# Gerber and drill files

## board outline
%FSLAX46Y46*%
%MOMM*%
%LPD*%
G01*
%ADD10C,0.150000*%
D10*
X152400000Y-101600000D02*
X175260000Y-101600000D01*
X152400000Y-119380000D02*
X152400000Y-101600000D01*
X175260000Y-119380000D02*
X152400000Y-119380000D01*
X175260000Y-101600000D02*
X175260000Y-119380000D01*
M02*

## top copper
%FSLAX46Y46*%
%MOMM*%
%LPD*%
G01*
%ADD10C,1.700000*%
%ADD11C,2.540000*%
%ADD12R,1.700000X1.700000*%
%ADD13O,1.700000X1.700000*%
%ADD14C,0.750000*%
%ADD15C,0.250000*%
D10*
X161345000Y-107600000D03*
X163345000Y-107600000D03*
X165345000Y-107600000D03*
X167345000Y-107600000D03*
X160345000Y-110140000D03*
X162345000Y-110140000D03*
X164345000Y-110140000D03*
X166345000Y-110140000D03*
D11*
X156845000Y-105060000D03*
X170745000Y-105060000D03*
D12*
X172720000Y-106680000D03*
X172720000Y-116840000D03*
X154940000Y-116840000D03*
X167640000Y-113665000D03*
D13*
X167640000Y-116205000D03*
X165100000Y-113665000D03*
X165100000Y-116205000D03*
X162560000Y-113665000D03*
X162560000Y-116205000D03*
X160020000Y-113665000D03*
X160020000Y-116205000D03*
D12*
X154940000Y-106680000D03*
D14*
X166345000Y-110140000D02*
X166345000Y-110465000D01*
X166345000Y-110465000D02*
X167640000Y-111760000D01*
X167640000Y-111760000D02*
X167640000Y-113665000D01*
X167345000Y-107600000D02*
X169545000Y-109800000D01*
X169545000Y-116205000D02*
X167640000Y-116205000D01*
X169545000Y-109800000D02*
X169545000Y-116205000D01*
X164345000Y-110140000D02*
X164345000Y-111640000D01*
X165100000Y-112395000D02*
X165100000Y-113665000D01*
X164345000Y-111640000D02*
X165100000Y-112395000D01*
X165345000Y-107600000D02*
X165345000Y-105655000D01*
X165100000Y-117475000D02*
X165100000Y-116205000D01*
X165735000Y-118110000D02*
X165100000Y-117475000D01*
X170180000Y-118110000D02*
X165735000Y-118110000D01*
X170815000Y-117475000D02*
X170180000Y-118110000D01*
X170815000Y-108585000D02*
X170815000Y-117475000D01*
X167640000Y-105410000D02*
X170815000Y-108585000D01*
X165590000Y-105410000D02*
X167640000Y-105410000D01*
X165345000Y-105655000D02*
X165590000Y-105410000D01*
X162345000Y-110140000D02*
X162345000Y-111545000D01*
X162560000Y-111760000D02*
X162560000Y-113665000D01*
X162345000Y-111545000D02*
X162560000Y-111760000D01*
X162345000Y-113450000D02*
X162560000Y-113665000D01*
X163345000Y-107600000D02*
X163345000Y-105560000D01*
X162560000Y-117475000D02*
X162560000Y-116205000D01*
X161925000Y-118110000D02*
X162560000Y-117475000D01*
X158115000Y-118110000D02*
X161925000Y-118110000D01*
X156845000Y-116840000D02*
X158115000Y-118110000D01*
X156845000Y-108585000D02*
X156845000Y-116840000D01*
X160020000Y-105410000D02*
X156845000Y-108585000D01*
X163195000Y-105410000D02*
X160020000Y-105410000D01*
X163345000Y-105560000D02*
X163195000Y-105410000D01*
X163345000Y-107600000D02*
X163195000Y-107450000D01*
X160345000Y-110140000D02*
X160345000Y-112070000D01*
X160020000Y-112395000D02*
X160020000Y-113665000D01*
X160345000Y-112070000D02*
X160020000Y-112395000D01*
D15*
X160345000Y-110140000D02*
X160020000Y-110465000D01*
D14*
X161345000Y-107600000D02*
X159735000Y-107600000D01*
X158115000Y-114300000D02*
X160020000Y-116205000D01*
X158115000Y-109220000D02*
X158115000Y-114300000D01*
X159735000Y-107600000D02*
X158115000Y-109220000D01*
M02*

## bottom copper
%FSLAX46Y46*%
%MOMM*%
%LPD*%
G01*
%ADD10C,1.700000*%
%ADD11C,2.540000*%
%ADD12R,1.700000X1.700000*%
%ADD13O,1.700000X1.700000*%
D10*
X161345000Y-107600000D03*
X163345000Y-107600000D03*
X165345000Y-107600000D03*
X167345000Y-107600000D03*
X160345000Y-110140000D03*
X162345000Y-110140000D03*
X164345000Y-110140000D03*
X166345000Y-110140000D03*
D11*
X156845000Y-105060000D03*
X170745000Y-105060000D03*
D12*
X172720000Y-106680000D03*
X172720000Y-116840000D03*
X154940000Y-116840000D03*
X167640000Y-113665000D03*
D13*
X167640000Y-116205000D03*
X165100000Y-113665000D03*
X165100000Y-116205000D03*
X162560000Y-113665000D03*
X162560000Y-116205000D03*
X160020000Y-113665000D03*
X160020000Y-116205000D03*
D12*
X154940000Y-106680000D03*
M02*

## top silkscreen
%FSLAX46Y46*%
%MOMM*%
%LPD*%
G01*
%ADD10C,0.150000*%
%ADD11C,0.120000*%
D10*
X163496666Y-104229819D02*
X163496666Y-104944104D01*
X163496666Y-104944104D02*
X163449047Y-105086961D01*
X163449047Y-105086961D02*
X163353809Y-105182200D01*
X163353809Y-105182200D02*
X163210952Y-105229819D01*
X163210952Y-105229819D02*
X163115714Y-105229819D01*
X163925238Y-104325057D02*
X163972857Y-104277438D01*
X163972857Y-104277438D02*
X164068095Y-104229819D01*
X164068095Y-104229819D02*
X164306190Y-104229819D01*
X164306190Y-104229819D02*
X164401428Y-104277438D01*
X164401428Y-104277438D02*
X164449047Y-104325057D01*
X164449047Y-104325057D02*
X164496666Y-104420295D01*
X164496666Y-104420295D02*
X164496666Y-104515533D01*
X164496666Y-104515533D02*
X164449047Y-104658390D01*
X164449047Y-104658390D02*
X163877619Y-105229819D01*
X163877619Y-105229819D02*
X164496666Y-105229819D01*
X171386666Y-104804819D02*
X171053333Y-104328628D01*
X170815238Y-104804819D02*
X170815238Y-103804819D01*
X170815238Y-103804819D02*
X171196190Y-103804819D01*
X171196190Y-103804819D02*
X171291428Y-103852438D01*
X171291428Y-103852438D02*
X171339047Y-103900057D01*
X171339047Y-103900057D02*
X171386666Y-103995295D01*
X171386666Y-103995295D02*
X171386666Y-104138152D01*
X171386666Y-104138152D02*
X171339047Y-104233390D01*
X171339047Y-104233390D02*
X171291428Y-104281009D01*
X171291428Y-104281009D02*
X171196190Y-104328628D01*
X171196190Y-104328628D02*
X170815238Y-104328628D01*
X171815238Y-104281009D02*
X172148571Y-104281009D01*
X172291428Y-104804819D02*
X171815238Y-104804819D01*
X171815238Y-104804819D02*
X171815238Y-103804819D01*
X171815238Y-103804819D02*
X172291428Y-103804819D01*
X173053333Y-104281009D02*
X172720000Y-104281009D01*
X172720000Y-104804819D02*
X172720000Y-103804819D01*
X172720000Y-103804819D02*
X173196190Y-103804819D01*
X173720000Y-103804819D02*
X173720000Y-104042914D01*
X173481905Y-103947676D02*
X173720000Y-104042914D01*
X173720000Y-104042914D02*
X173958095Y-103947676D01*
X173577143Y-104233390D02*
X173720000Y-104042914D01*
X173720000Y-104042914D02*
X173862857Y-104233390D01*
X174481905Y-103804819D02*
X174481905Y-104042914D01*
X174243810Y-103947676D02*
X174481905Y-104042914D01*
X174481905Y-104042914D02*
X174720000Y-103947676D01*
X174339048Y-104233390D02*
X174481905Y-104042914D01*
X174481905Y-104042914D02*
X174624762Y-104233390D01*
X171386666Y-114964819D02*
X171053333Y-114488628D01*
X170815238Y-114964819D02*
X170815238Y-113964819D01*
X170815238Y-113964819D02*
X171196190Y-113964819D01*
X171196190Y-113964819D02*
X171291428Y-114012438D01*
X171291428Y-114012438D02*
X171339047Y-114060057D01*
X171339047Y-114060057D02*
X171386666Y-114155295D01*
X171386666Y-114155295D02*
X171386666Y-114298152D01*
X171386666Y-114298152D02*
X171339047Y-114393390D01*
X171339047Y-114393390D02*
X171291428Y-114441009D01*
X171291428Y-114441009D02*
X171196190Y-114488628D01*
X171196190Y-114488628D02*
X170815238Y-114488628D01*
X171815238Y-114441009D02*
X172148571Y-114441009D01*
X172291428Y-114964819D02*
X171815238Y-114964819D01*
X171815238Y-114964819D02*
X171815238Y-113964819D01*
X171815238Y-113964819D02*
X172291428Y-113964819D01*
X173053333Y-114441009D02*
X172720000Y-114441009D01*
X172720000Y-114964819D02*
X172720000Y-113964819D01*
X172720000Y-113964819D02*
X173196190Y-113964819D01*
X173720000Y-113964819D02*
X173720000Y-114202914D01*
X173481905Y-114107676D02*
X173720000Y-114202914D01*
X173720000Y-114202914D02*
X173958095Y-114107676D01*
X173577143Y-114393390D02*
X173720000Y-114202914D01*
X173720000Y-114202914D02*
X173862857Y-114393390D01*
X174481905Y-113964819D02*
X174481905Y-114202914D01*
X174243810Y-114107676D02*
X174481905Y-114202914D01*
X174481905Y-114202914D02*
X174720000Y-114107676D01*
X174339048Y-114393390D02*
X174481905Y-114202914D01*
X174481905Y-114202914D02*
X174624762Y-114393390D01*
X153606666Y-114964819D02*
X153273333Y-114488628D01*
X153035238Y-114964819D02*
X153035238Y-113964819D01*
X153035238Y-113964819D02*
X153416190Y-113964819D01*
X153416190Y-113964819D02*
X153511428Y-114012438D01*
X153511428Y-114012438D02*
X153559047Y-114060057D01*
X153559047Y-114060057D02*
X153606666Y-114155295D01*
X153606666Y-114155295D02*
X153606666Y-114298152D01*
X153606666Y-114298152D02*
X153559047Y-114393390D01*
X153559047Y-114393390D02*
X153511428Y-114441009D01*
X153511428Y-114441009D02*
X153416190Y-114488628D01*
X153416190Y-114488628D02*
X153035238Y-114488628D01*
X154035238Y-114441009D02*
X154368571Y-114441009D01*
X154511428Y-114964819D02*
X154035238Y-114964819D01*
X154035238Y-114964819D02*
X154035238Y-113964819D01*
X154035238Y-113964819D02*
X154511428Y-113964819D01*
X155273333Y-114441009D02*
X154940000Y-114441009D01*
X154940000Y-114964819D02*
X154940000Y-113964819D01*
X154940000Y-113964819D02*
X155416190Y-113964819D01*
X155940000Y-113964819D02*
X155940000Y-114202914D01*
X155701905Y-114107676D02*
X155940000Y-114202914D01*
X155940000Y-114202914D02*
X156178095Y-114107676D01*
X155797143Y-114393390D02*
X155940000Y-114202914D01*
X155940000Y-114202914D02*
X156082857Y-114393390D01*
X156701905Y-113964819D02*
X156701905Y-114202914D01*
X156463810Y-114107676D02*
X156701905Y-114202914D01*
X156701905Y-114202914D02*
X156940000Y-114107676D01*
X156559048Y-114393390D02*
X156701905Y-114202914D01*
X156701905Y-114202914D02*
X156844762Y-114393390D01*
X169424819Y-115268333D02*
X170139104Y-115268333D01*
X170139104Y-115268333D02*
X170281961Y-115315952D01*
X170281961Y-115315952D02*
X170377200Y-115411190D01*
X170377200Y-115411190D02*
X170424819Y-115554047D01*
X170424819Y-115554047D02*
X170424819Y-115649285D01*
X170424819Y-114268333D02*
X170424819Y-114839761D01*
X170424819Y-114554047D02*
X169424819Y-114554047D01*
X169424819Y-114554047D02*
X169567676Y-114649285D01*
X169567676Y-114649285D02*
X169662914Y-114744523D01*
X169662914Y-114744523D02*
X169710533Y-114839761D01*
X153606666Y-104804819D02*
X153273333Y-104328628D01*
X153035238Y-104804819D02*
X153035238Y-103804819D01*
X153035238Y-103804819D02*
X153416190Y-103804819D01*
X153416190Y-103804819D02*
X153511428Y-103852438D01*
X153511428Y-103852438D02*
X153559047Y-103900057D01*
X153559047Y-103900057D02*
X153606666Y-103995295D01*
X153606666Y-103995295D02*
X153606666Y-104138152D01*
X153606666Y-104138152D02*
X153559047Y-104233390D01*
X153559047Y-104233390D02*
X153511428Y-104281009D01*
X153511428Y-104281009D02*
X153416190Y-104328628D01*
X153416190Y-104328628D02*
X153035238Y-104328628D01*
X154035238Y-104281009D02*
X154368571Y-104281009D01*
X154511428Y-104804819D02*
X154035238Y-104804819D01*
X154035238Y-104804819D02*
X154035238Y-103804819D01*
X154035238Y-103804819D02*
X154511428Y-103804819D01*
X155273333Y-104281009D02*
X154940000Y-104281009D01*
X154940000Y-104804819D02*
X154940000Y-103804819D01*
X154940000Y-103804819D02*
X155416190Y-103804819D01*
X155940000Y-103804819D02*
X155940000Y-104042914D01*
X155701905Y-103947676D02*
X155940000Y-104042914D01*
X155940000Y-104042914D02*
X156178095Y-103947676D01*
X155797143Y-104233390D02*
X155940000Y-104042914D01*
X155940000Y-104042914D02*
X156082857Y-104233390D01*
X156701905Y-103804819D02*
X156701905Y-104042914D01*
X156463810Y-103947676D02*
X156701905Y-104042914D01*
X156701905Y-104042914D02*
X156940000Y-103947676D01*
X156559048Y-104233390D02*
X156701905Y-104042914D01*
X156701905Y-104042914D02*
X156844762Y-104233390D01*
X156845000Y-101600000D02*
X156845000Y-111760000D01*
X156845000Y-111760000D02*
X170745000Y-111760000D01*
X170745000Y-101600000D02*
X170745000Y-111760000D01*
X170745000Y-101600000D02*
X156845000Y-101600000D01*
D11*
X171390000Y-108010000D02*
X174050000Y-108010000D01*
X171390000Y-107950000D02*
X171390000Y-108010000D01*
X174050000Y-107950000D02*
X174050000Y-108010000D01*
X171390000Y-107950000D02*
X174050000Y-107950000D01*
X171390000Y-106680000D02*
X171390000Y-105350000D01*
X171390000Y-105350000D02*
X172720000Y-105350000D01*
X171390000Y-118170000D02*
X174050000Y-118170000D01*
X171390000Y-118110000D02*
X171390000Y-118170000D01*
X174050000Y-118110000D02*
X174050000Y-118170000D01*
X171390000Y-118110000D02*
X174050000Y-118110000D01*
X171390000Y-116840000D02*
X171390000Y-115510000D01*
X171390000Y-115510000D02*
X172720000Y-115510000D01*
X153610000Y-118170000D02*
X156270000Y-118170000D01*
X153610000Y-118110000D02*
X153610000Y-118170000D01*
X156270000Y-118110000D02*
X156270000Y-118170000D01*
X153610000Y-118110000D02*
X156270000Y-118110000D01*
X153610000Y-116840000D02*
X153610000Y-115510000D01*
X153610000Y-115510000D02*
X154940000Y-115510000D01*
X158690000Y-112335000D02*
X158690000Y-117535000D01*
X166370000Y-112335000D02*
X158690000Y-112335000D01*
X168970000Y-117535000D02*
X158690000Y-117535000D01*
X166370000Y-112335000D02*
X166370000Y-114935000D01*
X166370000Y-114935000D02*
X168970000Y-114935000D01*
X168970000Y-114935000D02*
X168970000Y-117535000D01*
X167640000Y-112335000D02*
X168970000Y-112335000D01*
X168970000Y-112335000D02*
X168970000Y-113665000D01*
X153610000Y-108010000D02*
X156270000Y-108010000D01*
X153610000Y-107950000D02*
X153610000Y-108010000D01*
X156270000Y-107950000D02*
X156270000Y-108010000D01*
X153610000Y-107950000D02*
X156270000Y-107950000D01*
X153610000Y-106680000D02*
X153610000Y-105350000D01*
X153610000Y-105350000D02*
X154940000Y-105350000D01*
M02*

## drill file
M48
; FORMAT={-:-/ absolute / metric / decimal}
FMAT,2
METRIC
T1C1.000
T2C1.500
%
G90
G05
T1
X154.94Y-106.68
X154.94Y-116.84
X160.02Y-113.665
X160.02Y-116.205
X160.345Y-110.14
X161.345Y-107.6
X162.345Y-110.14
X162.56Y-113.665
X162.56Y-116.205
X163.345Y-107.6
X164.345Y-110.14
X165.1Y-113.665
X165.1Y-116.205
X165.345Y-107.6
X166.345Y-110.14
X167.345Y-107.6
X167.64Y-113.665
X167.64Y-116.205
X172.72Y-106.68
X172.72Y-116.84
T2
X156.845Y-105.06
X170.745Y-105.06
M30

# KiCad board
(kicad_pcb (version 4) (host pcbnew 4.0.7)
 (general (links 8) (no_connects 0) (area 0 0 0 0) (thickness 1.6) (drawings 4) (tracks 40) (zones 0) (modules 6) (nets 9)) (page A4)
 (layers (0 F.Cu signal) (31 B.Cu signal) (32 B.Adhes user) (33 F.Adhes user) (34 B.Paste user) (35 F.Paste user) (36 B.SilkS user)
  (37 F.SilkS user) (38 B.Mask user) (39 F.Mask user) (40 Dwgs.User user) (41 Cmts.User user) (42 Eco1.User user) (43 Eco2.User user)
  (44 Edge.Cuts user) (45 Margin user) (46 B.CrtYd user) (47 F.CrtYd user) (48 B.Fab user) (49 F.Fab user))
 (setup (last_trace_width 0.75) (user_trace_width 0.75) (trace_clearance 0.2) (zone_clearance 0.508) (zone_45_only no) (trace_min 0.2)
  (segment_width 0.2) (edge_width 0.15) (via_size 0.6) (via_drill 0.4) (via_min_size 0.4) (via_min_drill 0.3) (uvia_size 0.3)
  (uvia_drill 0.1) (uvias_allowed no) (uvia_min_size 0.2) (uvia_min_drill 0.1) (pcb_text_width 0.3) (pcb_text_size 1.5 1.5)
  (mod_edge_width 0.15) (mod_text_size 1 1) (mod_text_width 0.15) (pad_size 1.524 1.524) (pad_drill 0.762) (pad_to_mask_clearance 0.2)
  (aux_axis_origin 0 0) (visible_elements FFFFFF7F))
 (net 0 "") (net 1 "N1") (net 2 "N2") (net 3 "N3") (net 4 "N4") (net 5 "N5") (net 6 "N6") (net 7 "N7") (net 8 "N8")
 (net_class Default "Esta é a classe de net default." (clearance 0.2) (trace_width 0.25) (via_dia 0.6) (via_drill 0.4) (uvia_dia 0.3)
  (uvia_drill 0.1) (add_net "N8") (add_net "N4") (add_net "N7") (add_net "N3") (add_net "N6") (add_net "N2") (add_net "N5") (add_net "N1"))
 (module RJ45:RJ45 (layer F.Cu) (at 156.845 101.6)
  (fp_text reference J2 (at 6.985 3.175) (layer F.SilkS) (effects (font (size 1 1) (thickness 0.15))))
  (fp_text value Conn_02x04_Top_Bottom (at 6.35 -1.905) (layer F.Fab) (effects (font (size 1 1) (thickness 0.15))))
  (fp_line (start 0 0) (end 0 10.16) (layer F.SilkS) (width 0.15))
  (fp_line (start 0 10.16) (end 13.9 10.16) (layer F.SilkS) (width 0.15))
  (fp_line (start 13.9 0) (end 13.9 10.16) (layer F.SilkS) (width 0.15))
  (fp_line (start 13.9 0) (end 0 0) (layer F.SilkS) (width 0.15))
  (pad 1 thru_hole circle (at 4.5 6) (size 1.7 1.7) (drill 1) (layers *.Cu *.Mask) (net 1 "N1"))
  (pad 2 thru_hole circle (at 6.5 6) (size 1.7 1.7) (drill 1) (layers *.Cu *.Mask) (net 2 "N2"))
  (pad 3 thru_hole circle (at 8.5 6) (size 1.7 1.7) (drill 1) (layers *.Cu *.Mask) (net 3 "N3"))
  (pad 4 thru_hole circle (at 10.5 6) (size 1.7 1.7) (drill 1) (layers *.Cu *.Mask) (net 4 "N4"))
  (pad 5 thru_hole circle (at 3.5 8.54) (size 1.7 1.7) (drill 1) (layers *.Cu *.Mask) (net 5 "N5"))
  (pad 6 thru_hole circle (at 5.5 8.54) (size 1.7 1.7) (drill 1) (layers *.Cu *.Mask) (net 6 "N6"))
  (pad 7 thru_hole circle (at 7.5 8.54) (size 1.7 1.7) (drill 1) (layers *.Cu *.Mask) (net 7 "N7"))
  (pad 8 thru_hole circle (at 9.5 8.54) (size 1.7 1.7) (drill 1) (layers *.Cu *.Mask) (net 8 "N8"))
  (pad 9 thru_hole circle (at 0 3.46) (size 2.54 2.54) (drill 1.5) (layers *.Cu *.Mask))
  (pad 10 thru_hole circle (at 13.9 3.46) (size 2.54 2.54) (drill 1.5) (layers *.Cu *.Mask)))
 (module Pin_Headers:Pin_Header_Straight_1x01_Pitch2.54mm (layer F.Cu) (at 172.72 106.68)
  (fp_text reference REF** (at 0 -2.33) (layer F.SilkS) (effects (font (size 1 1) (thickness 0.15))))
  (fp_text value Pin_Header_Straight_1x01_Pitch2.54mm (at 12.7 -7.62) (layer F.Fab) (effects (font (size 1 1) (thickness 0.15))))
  (fp_line (start -1.33 1.33) (end 1.33 1.33) (layer F.SilkS) (width 0.12))
  (fp_line (start -1.33 1.27) (end -1.33 1.33) (layer F.SilkS) (width 0.12))
  (fp_line (start 1.33 1.27) (end 1.33 1.33) (layer F.SilkS) (width 0.12))
  (fp_line (start -1.33 1.27) (end 1.33 1.27) (layer F.SilkS) (width 0.12))
  (fp_line (start -1.33 0) (end -1.33 -1.33) (layer F.SilkS) (width 0.12))
  (fp_line (start -1.33 -1.33) (end 0 -1.33) (layer F.SilkS) (width 0.12))
  (pad 1 thru_hole rect (at 0 0) (size 1.7 1.7) (drill 1) (layers *.Cu *.Mask)))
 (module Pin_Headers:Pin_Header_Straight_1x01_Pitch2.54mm (layer F.Cu) (at 172.72 116.84)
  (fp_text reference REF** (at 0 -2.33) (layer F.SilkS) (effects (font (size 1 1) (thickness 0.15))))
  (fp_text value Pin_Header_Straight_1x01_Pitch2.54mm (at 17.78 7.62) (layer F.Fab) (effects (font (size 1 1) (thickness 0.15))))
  (fp_line (start -1.33 1.33) (end 1.33 1.33) (layer F.SilkS) (width 0.12))
  (fp_line (start -1.33 1.27) (end -1.33 1.33) (layer F.SilkS) (width 0.12))
  (fp_line (start 1.33 1.27) (end 1.33 1.33) (layer F.SilkS) (width 0.12))
  (fp_line (start -1.33 1.27) (end 1.33 1.27) (layer F.SilkS) (width 0.12))
  (fp_line (start -1.33 0) (end -1.33 -1.33) (layer F.SilkS) (width 0.12))
  (fp_line (start -1.33 -1.33) (end 0 -1.33) (layer F.SilkS) (width 0.12))
  (pad 1 thru_hole rect (at 0 0) (size 1.7 1.7) (drill 1) (layers *.Cu *.Mask)))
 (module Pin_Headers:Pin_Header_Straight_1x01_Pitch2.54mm (layer F.Cu) (at 154.94 116.84)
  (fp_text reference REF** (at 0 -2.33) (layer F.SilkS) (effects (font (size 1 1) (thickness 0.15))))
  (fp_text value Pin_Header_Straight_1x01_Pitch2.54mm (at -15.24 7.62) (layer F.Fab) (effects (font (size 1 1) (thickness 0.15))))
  (fp_line (start -1.33 1.33) (end 1.33 1.33) (layer F.SilkS) (width 0.12))
  (fp_line (start -1.33 1.27) (end -1.33 1.33) (layer F.SilkS) (width 0.12))
  (fp_line (start 1.33 1.27) (end 1.33 1.33) (layer F.SilkS) (width 0.12))
  (fp_line (start -1.33 1.27) (end 1.33 1.27) (layer F.SilkS) (width 0.12))
  (fp_line (start -1.33 0) (end -1.33 -1.33) (layer F.SilkS) (width 0.12))
  (fp_line (start -1.33 -1.33) (end 0 -1.33) (layer F.SilkS) (width 0.12))
  (pad 1 thru_hole rect (at 0 0) (size 1.7 1.7) (drill 1) (layers *.Cu *.Mask)))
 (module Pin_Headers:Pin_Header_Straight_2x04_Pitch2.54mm (layer F.Cu) (at 167.64 113.665 270)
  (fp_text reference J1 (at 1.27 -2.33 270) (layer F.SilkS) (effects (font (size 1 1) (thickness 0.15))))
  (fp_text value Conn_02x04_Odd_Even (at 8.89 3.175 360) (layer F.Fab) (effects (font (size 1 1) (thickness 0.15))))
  (fp_line (start -1.33 8.95) (end 3.87 8.95) (layer F.SilkS) (width 0.12))
  (fp_line (start -1.33 1.27) (end -1.33 8.95) (layer F.SilkS) (width 0.12))
  (fp_line (start 3.87 -1.33) (end 3.87 8.95) (layer F.SilkS) (width 0.12))
  (fp_line (start -1.33 1.27) (end 1.27 1.27) (layer F.SilkS) (width 0.12))
  (fp_line (start 1.27 1.27) (end 1.27 -1.33) (layer F.SilkS) (width 0.12))
  (fp_line (start 1.27 -1.33) (end 3.87 -1.33) (layer F.SilkS) (width 0.12))
  (fp_line (start -1.33 0) (end -1.33 -1.33) (layer F.SilkS) (width 0.12))
  (fp_line (start -1.33 -1.33) (end 0 -1.33) (layer F.SilkS) (width 0.12))
  (pad 1 thru_hole rect (at 0 0 270) (size 1.7 1.7) (drill 1) (layers *.Cu *.Mask) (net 8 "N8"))
  (pad 2 thru_hole oval (at 2.54 0 270) (size 1.7 1.7) (drill 1) (layers *.Cu *.Mask) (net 4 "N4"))
  (pad 3 thru_hole oval (at 0 2.54 270) (size 1.7 1.7) (drill 1) (layers *.Cu *.Mask) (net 7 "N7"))
  (pad 4 thru_hole oval (at 2.54 2.54 270) (size 1.7 1.7) (drill 1) (layers *.Cu *.Mask) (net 3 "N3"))
  (pad 5 thru_hole oval (at 0 5.08 270) (size 1.7 1.7) (drill 1) (layers *.Cu *.Mask) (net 6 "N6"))
  (pad 6 thru_hole oval (at 2.54 5.08 270) (size 1.7 1.7) (drill 1) (layers *.Cu *.Mask) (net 2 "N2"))
  (pad 7 thru_hole oval (at 0 7.62 270) (size 1.7 1.7) (drill 1) (layers *.Cu *.Mask) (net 5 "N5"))
  (pad 8 thru_hole oval (at 2.54 7.62 270) (size 1.7 1.7) (drill 1) (layers *.Cu *.Mask) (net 1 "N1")))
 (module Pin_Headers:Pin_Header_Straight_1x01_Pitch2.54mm (layer F.Cu) (at 154.94 106.68)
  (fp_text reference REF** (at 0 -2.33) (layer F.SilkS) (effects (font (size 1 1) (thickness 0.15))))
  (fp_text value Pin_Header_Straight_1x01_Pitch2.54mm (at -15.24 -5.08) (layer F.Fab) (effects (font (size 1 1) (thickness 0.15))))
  (fp_line (start -1.33 1.33) (end 1.33 1.33) (layer F.SilkS) (width 0.12))
  (fp_line (start -1.33 1.27) (end -1.33 1.33) (layer F.SilkS) (width 0.12))
  (fp_line (start 1.33 1.27) (end 1.33 1.33) (layer F.SilkS) (width 0.12))
  (fp_line (start -1.33 1.27) (end 1.33 1.27) (layer F.SilkS) (width 0.12))
  (fp_line (start -1.33 0) (end -1.33 -1.33) (layer F.SilkS) (width 0.12))
  (fp_line (start -1.33 -1.33) (end 0 -1.33) (layer F.SilkS) (width 0.12))
  (pad 1 thru_hole rect (at 0 0) (size 1.7 1.7) (drill 1) (layers *.Cu *.Mask)))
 (gr_line (start 152.4 101.6) (end 175.26 101.6) (angle 90) (layer Edge.Cuts) (width 0.15))
 (gr_line (start 152.4 119.38) (end 152.4 101.6) (angle 90) (layer Edge.Cuts) (width 0.15))
 (gr_line (start 175.26 119.38) (end 152.4 119.38) (angle 90) (layer Edge.Cuts) (width 0.15))
 (gr_line (start 175.26 101.6) (end 175.26 119.38) (angle 90) (layer Edge.Cuts) (width 0.15))
 (segment (start 166.345 110.14) (end 166.345 110.465) (width 0.75) (layer F.Cu) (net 8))
 (segment (start 166.345 110.465) (end 167.64 111.76) (width 0.75) (layer F.Cu) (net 8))
 (segment (start 167.64 111.76) (end 167.64 113.665) (width 0.75) (layer F.Cu) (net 8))
 (segment (start 167.345 107.6) (end 169.545 109.8) (width 0.75) (layer F.Cu) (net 4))
 (segment (start 169.545 116.205) (end 167.64 116.205) (width 0.75) (layer F.Cu) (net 4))
 (segment (start 169.545 109.8) (end 169.545 116.205) (width 0.75) (layer F.Cu) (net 4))
 (segment (start 164.345 110.14) (end 164.345 111.64) (width 0.75) (layer F.Cu) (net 7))
 (segment (start 165.1 112.395) (end 165.1 113.665) (width 0.75) (layer F.Cu) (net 7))
 (segment (start 164.345 111.64) (end 165.1 112.395) (width 0.75) (layer F.Cu) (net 7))
 (segment (start 165.345 107.6) (end 165.345 105.655) (width 0.75) (layer F.Cu) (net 3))
 (segment (start 165.1 117.475) (end 165.1 116.205) (width 0.75) (layer F.Cu) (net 3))
 (segment (start 165.735 118.11) (end 165.1 117.475) (width 0.75) (layer F.Cu) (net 3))
 (segment (start 170.18 118.11) (end 165.735 118.11) (width 0.75) (layer F.Cu) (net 3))
 (segment (start 170.815 117.475) (end 170.18 118.11) (width 0.75) (layer F.Cu) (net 3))
 (segment (start 170.815 108.585) (end 170.815 117.475) (width 0.75) (layer F.Cu) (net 3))
 (segment (start 167.64 105.41) (end 170.815 108.585) (width 0.75) (layer F.Cu) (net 3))
 (segment (start 165.59 105.41) (end 167.64 105.41) (width 0.75) (layer F.Cu) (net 3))
 (segment (start 165.345 105.655) (end 165.59 105.41) (width 0.75) (layer F.Cu) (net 3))
 (segment (start 162.345 110.14) (end 162.345 111.545) (width 0.75) (layer F.Cu) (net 6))
 (segment (start 162.56 111.76) (end 162.56 113.665) (width 0.75) (layer F.Cu) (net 6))
 (segment (start 162.345 111.545) (end 162.56 111.76) (width 0.75) (layer F.Cu) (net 6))
 (segment (start 162.345 113.45) (end 162.56 113.665) (width 0.75) (layer F.Cu) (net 6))
 (segment (start 163.345 107.6) (end 163.345 105.56) (width 0.75) (layer F.Cu) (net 2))
 (segment (start 162.56 117.475) (end 162.56 116.205) (width 0.75) (layer F.Cu) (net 2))
 (segment (start 161.925 118.11) (end 162.56 117.475) (width 0.75) (layer F.Cu) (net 2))
 (segment (start 158.115 118.11) (end 161.925 118.11) (width 0.75) (layer F.Cu) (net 2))
 (segment (start 156.845 116.84) (end 158.115 118.11) (width 0.75) (layer F.Cu) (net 2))
 (segment (start 156.845 108.585) (end 156.845 116.84) (width 0.75) (layer F.Cu) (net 2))
 (segment (start 160.02 105.41) (end 156.845 108.585) (width 0.75) (layer F.Cu) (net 2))
 (segment (start 163.195 105.41) (end 160.02 105.41) (width 0.75) (layer F.Cu) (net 2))
 (segment (start 163.345 105.56) (end 163.195 105.41) (width 0.75) (layer F.Cu) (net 2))
 (segment (start 163.345 107.6) (end 163.195 107.45) (width 0.75) (layer F.Cu) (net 2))
 (segment (start 160.345 110.14) (end 160.345 112.07) (width 0.75) (layer F.Cu) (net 5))
 (segment (start 160.02 112.395) (end 160.02 113.665) (width 0.75) (layer F.Cu) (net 5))
 (segment (start 160.345 112.07) (end 160.02 112.395) (width 0.75) (layer F.Cu) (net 5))
 (segment (start 160.345 110.14) (end 160.02 110.465) (width 0.25) (layer F.Cu) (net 5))
 (segment (start 161.345 107.6) (end 159.735 107.6) (width 0.75) (layer F.Cu) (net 1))
 (segment (start 158.115 114.3) (end 160.02 116.205) (width 0.75) (layer F.Cu) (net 1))
 (segment (start 158.115 109.22) (end 158.115 114.3) (width 0.75) (layer F.Cu) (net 1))
 (segment (start 159.735 107.6) (end 158.115 109.22) (width 0.75) (layer F.Cu) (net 1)))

